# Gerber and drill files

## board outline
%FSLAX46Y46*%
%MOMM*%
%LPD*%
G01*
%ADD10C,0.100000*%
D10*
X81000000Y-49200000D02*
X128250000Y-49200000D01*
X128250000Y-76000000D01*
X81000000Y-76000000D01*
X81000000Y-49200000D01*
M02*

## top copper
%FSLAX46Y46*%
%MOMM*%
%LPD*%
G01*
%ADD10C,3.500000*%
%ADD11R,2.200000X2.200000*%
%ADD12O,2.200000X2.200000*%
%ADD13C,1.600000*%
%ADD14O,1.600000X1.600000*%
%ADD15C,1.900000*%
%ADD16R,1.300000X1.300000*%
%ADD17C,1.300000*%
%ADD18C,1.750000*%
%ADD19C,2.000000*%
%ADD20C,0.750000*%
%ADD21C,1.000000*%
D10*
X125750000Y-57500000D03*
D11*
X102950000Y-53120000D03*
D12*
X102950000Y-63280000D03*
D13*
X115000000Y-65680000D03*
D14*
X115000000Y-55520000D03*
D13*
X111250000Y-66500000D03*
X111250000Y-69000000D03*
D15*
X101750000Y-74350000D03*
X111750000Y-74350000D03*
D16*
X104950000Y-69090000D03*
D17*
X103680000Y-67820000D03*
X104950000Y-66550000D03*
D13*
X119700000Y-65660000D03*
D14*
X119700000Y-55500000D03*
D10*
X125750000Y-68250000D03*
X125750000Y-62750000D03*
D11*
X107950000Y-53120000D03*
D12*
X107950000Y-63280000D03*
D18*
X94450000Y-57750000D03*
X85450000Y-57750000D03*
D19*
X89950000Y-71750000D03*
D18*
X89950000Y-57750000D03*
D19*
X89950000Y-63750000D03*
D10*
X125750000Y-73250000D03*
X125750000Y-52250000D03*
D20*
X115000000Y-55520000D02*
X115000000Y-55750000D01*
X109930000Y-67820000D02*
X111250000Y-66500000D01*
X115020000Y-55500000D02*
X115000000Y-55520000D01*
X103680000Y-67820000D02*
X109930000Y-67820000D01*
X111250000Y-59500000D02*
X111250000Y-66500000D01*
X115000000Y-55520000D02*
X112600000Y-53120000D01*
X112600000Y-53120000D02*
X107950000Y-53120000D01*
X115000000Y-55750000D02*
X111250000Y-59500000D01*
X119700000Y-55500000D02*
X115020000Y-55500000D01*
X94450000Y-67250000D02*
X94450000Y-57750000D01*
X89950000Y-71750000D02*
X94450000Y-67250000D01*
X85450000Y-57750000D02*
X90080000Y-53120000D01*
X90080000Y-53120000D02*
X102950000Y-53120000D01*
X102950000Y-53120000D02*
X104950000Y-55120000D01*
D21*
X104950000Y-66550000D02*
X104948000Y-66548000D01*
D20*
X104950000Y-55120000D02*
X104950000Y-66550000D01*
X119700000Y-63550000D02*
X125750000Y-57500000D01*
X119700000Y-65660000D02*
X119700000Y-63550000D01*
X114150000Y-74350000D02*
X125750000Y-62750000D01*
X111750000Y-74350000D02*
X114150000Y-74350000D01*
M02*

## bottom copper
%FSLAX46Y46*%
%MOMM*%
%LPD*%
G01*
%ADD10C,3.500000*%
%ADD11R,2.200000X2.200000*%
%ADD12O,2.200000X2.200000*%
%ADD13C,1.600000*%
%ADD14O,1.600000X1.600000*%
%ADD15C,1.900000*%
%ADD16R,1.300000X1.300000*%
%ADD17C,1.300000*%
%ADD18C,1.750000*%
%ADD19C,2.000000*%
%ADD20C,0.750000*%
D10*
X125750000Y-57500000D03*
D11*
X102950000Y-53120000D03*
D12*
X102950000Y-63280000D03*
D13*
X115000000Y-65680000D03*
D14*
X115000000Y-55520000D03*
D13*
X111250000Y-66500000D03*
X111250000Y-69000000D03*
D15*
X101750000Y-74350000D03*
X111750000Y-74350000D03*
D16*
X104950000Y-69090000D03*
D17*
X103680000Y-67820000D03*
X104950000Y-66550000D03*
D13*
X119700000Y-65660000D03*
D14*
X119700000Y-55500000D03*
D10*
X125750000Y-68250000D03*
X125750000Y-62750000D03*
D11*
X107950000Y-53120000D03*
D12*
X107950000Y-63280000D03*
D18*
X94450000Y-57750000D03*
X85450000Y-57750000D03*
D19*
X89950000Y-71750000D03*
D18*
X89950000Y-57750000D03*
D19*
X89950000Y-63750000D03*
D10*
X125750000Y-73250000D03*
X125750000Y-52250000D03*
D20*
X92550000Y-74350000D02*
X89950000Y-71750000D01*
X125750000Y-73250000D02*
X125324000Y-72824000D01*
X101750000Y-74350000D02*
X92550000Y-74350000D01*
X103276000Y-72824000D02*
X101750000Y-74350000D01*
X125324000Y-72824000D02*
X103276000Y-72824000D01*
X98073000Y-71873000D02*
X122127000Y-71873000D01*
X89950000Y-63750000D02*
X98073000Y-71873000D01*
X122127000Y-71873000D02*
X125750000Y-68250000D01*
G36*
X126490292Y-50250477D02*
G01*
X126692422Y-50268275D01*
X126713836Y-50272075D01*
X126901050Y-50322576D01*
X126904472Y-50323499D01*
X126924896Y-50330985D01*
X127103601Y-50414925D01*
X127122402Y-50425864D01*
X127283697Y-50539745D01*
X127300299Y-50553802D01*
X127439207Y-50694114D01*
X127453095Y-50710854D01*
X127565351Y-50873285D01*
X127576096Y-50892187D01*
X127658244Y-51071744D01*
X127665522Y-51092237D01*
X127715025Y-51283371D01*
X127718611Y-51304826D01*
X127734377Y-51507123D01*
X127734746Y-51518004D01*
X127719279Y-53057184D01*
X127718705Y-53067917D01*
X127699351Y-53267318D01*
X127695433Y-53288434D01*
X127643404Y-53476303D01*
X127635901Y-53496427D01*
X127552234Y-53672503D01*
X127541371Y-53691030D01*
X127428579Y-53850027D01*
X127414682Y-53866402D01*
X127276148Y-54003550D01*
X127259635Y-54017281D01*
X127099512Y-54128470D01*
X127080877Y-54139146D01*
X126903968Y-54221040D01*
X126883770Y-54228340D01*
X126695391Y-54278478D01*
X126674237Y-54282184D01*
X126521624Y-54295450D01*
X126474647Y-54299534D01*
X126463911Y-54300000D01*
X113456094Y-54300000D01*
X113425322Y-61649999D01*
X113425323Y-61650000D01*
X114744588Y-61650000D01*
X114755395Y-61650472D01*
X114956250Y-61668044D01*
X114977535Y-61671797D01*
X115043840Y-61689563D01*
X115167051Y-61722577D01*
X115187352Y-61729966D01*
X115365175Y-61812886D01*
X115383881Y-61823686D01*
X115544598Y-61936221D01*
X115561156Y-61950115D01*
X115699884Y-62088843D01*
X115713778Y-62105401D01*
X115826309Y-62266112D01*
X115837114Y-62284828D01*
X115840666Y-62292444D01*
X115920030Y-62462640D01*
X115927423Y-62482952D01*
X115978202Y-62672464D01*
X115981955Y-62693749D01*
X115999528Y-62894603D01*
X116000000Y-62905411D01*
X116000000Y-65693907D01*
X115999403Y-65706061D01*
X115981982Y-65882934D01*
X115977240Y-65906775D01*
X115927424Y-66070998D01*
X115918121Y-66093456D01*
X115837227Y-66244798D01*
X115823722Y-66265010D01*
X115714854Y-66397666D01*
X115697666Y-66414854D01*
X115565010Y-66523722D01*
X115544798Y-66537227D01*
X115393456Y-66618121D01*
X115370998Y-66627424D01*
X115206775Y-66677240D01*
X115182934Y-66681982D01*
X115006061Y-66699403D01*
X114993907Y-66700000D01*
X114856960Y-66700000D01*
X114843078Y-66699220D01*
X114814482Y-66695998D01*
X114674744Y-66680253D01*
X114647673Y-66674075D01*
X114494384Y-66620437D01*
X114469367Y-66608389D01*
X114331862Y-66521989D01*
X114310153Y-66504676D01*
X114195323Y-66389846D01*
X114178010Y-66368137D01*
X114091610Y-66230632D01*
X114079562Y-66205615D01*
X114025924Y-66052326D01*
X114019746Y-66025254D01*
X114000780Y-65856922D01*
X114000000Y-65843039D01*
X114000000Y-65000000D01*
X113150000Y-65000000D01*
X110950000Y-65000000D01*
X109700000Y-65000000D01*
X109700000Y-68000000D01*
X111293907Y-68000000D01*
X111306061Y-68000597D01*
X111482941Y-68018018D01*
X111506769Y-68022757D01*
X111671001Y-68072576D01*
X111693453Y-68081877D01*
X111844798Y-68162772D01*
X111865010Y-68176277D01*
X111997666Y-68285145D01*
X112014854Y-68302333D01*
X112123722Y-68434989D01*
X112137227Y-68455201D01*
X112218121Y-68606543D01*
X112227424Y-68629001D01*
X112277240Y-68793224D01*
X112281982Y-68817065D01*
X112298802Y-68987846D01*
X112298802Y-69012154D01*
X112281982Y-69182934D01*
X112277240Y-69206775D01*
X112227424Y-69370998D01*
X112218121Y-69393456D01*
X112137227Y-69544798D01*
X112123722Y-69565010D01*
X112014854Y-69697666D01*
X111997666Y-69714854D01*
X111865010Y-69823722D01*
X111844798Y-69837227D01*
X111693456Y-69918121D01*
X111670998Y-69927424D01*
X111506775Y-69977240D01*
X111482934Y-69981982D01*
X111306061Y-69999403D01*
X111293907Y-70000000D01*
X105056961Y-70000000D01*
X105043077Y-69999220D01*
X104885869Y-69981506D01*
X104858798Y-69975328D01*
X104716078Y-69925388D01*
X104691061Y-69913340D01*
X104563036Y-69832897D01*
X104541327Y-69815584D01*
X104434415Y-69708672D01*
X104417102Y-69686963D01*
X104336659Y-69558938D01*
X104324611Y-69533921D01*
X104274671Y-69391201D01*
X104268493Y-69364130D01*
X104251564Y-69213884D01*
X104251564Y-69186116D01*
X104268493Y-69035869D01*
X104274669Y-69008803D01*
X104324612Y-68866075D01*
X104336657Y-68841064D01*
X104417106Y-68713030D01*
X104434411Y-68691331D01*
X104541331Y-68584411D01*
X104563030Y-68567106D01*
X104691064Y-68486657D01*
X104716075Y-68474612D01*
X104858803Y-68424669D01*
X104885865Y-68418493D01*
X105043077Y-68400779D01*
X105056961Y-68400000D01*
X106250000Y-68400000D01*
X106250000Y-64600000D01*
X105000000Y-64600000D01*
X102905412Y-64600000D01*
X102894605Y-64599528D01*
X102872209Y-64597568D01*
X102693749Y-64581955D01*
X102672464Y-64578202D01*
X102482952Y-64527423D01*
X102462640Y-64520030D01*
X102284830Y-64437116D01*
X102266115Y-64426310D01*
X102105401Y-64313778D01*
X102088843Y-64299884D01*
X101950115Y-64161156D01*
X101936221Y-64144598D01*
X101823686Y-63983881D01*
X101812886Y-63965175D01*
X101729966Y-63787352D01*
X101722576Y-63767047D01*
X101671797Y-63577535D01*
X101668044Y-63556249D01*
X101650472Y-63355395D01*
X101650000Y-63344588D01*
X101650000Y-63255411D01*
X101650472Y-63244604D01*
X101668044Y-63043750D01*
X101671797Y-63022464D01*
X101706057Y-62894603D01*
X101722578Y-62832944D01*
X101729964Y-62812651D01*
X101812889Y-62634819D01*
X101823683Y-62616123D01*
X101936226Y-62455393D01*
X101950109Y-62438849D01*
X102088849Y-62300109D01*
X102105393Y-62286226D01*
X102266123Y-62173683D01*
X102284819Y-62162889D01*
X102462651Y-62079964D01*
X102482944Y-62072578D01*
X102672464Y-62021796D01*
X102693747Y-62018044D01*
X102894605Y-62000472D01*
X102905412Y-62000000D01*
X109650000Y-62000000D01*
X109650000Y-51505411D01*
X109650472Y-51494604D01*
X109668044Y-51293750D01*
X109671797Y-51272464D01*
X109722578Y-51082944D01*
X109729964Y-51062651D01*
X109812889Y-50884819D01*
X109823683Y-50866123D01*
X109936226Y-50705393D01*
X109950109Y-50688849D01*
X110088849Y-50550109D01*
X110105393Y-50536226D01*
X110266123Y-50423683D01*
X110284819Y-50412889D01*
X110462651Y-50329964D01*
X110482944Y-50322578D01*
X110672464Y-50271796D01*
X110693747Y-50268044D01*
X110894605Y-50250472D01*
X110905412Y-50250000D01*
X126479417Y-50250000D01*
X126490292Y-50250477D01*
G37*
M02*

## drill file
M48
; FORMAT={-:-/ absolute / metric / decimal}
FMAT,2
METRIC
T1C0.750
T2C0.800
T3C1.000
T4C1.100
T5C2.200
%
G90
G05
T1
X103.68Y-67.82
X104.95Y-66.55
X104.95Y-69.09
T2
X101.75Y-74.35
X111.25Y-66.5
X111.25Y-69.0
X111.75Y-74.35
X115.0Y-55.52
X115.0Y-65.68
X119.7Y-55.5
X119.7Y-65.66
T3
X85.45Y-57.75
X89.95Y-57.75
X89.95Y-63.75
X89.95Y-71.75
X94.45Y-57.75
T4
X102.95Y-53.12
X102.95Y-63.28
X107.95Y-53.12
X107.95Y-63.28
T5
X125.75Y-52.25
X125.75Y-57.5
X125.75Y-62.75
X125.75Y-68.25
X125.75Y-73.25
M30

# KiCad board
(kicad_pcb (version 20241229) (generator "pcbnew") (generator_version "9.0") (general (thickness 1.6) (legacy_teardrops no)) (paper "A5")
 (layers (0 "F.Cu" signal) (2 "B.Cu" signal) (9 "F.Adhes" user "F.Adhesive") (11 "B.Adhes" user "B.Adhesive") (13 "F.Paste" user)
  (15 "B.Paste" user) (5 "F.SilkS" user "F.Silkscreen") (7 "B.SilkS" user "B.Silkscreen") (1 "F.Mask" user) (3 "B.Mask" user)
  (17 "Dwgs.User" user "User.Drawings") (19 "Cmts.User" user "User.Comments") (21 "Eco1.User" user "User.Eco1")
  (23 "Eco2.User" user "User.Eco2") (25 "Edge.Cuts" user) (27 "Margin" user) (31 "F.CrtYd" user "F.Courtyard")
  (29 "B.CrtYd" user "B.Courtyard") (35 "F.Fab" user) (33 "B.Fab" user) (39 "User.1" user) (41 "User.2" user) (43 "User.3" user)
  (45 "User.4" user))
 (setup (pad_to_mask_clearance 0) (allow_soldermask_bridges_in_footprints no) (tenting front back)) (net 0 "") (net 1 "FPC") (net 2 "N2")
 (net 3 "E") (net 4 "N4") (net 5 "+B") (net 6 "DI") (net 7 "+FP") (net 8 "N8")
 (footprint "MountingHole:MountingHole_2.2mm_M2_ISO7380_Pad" (layer "F.Cu") (at 125.75 57.5 90)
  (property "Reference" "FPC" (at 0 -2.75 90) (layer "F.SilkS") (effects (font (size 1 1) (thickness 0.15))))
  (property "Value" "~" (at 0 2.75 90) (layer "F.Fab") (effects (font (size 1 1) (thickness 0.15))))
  (pad "1" thru_hole circle (at 0 0 90) (size 3.5 3.5) (drill 2.2) (layers "*.Cu" "*.Mask") (remove_unused_layers no) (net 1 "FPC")))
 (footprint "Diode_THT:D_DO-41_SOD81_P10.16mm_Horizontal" (layer "F.Cu") (at 102.95 53.12 -90)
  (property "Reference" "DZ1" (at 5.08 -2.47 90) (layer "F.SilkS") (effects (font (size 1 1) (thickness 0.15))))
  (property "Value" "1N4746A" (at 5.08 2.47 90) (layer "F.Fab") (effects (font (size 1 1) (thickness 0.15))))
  (pad "1" thru_hole rect (at 0 0 270) (size 2.2 2.2) (drill 1.1) (layers "*.Cu" "*.Mask") (remove_unused_layers no) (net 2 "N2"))
  (pad "2" thru_hole oval (at 10.16 0 270) (size 2.2 2.2) (drill 1.1) (layers "*.Cu" "*.Mask") (remove_unused_layers no) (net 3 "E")))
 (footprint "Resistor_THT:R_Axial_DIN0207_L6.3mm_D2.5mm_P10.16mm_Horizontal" (layer "F.Cu") (at 115 65.68 90)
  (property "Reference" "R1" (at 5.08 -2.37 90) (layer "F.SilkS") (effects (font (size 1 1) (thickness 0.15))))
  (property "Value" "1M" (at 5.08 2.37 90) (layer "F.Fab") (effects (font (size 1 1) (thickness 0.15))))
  (pad "1" thru_hole circle (at 0 0 90) (size 1.6 1.6) (drill 0.8) (layers "*.Cu" "*.Mask") (remove_unused_layers no) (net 3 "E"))
  (pad "2" thru_hole oval (at 10.16 0 90) (size 1.6 1.6) (drill 0.8) (layers "*.Cu" "*.Mask") (remove_unused_layers no) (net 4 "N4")))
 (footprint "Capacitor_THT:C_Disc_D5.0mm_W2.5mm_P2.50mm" (layer "F.Cu") (at 111.25 66.5 -90)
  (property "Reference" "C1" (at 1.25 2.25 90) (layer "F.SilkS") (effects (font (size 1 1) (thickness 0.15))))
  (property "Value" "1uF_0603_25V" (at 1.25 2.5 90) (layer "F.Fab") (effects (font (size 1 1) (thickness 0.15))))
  (pad "1" thru_hole circle (at 0 0 270) (size 1.6 1.6) (drill 0.8) (layers "*.Cu" "*.Mask") (remove_unused_layers no) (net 4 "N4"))
  (pad "2" thru_hole circle (at 2.5 0 270) (size 1.6 1.6) (drill 0.8) (layers "*.Cu" "*.Mask") (remove_unused_layers no) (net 3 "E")))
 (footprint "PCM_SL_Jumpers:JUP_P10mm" (layer "F.Cu") (at 106.75 74.35)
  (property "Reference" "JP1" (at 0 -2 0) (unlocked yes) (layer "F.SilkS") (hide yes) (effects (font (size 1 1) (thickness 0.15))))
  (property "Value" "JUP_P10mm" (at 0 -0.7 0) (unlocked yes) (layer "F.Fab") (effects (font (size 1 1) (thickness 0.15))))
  (pad "1" thru_hole circle (at -5 0) (size 1.9 1.9) (drill 0.8) (layers "*.Cu" "*.Mask") (remove_unused_layers no) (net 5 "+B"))
  (pad "2" thru_hole circle (at 5 0) (size 1.9 1.9) (drill 0.8) (layers "*.Cu" "*.Mask") (remove_unused_layers no) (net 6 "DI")))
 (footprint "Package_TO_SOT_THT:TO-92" (layer "F.Cu") (at 104.95 69.09 90)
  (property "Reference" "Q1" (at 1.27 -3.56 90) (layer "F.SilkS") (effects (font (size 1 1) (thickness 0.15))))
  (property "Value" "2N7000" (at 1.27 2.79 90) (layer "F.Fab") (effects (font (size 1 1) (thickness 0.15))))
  (pad "1" thru_hole rect (at 0 0 90) (size 1.3 1.3) (drill 0.75) (layers "*.Cu" "*.Mask") (remove_unused_layers no) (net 3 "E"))
  (pad "2" thru_hole circle (at 1.27 -1.27 90) (size 1.3 1.3) (drill 0.75) (layers "*.Cu" "*.Mask") (remove_unused_layers no) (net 4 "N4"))
  (pad "3" thru_hole circle (at 2.54 0 90) (size 1.3 1.3) (drill 0.75) (layers "*.Cu" "*.Mask") (remove_unused_layers no) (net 2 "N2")))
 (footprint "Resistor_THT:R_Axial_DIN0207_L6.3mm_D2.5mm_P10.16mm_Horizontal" (layer "F.Cu") (at 119.7 65.66 90)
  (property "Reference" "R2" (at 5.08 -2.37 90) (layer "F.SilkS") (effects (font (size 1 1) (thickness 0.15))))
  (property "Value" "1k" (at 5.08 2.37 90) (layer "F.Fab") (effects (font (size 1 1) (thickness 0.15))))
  (pad "1" thru_hole circle (at 0 0 90) (size 1.6 1.6) (drill 0.8) (layers "*.Cu" "*.Mask") (remove_unused_layers no) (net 1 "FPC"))
  (pad "2" thru_hole oval (at 10.16 0 90) (size 1.6 1.6) (drill 0.8) (layers "*.Cu" "*.Mask") (remove_unused_layers no) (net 4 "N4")))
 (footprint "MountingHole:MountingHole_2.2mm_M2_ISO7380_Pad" (layer "F.Cu") (at 125.75 68.25 90)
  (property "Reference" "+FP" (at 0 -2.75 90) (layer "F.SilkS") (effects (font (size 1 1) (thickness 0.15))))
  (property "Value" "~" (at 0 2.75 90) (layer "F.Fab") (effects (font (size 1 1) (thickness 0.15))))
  (pad "1" thru_hole circle (at 0 0 90) (size 3.5 3.5) (drill 2.2) (layers "*.Cu" "*.Mask") (remove_unused_layers no) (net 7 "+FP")))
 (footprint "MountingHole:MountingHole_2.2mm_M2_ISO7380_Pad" (layer "F.Cu") (at 125.75 62.75 90)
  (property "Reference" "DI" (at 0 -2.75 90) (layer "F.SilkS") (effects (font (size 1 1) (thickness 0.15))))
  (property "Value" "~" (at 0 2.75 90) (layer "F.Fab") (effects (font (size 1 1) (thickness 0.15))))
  (pad "1" thru_hole circle (at 0 0 90) (size 3.5 3.5) (drill 2.2) (layers "*.Cu" "*.Mask") (remove_unused_layers no) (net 6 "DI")))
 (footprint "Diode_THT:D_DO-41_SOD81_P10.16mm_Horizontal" (layer "F.Cu") (at 107.95 53.12 -90)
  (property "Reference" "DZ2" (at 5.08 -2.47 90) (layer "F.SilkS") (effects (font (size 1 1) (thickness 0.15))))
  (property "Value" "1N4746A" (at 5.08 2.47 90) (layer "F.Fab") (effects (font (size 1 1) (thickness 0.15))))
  (pad "1" thru_hole rect (at 0 0 270) (size 2.2 2.2) (drill 1.1) (layers "*.Cu" "*.Mask") (remove_unused_layers no) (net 4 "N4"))
  (pad "2" thru_hole oval (at 10.16 0 270) (size 2.2 2.2) (drill 1.1) (layers "*.Cu" "*.Mask") (remove_unused_layers no) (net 3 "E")))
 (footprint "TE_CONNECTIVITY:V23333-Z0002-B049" (layer "F.Cu") (at 89.95 63.75)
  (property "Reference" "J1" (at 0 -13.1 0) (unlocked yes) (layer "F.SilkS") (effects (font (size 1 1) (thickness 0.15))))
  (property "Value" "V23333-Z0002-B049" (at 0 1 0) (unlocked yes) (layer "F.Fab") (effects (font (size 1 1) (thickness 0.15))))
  (pad "1" thru_hole circle (at 4.5 -6) (size 1.75 1.75) (drill 1) (layers "*.Cu" "*.Mask") (remove_unused_layers no) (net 5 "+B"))
  (pad "2" thru_hole circle (at -4.5 -6) (size 1.75 1.75) (drill 1) (layers "*.Cu" "*.Mask") (remove_unused_layers no) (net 2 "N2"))
  (pad "3" thru_hole circle (at 0 8) (size 2 2) (drill 1) (layers "*.Cu" "*.Mask") (remove_unused_layers no) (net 5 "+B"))
  (pad "4" thru_hole circle (at 0 -6) (size 1.75 1.75) (drill 1) (layers "*.Cu" "*.Mask") (remove_unused_layers no) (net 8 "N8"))
  (pad "5" thru_hole circle (at 0 0) (size 2 2) (drill 1) (layers "*.Cu" "*.Mask") (remove_unused_layers no) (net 7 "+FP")))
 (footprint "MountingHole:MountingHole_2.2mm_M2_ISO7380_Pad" (layer "F.Cu") (at 125.75 73.25 90)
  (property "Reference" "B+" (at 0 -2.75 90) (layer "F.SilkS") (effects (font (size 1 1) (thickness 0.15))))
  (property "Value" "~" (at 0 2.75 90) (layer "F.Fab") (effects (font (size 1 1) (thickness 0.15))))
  (pad "1" thru_hole circle (at 0 0 90) (size 3.5 3.5) (drill 2.2) (layers "*.Cu" "*.Mask") (remove_unused_layers no) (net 5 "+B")))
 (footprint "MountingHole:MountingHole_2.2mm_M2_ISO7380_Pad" (layer "F.Cu") (at 125.75 52.25 90)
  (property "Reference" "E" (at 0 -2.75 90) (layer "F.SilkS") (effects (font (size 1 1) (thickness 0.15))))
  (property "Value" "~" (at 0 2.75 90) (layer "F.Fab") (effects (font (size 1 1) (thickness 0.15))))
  (pad "1" thru_hole circle (at 0 0 90) (size 3.5 3.5) (drill 2.2) (layers "*.Cu" "*.Mask") (remove_unused_layers no) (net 3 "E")))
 (gr_rect (start 81 49.2) (end 128.25 76) (stroke (width 0.1) (type default)) (fill no) (layer "Edge.Cuts"))
 (segment (start 115 55.52) (end 115 55.75) (width 0.75) (layer "F.Cu") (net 4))
 (segment (start 109.93 67.82) (end 111.25 66.5) (width 0.75) (layer "F.Cu") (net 4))
 (segment (start 115.02 55.5) (end 115 55.52) (width 0.75) (layer "F.Cu") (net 4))
 (segment (start 103.68 67.82) (end 109.93 67.82) (width 0.75) (layer "F.Cu") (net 4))
 (segment (start 111.25 59.5) (end 111.25 66.5) (width 0.75) (layer "F.Cu") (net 4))
 (segment (start 115 55.52) (end 112.6 53.12) (width 0.75) (layer "F.Cu") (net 4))
 (segment (start 112.6 53.12) (end 107.95 53.12) (width 0.75) (layer "F.Cu") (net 4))
 (segment (start 115 55.75) (end 111.25 59.5) (width 0.75) (layer "F.Cu") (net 4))
 (segment (start 119.7 55.5) (end 115.02 55.5) (width 0.75) (layer "F.Cu") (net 4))
 (segment (start 94.45 67.25) (end 94.45 57.75) (width 0.75) (layer "F.Cu") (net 5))
 (segment (start 89.95 71.75) (end 94.45 67.25) (width 0.75) (layer "F.Cu") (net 5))
 (segment (start 92.55 74.35) (end 89.95 71.75) (width 0.75) (layer "B.Cu") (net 5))
 (segment (start 125.75 73.25) (end 125.324 72.824) (width 0.75) (layer "B.Cu") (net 5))
 (segment (start 101.75 74.35) (end 92.55 74.35) (width 0.75) (layer "B.Cu") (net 5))
 (segment (start 103.276 72.824) (end 101.75 74.35) (width 0.75) (layer "B.Cu") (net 5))
 (segment (start 125.324 72.824) (end 103.276 72.824) (width 0.75) (layer "B.Cu") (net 5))
 (segment (start 85.45 57.75) (end 90.08 53.12) (width 0.75) (layer "F.Cu") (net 2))
 (segment (start 90.08 53.12) (end 102.95 53.12) (width 0.75) (layer "F.Cu") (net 2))
 (segment (start 102.95 53.12) (end 104.95 55.12) (width 0.75) (layer "F.Cu") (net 2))
 (segment (start 104.95 66.55) (end 104.948 66.548) (width 1) (layer "F.Cu") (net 2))
 (segment (start 104.95 55.12) (end 104.95 66.55) (width 0.75) (layer "F.Cu") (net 2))
 (segment (start 98.073 71.873) (end 122.127 71.873) (width 0.75) (layer "B.Cu") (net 7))
 (segment (start 89.95 63.75) (end 98.073 71.873) (width 0.75) (layer "B.Cu") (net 7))
 (segment (start 122.127 71.873) (end 125.75 68.25) (width 0.75) (layer "B.Cu") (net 7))
 (segment (start 119.7 63.55) (end 125.75 57.5) (width 0.75) (layer "F.Cu") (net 1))
 (segment (start 119.7 65.66) (end 119.7 63.55) (width 0.75) (layer "F.Cu") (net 1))
 (segment (start 114.15 74.35) (end 125.75 62.75) (width 0.75) (layer "F.Cu") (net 6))
 (segment (start 111.75 74.35) (end 114.15 74.35) (width 0.75) (layer "F.Cu") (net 6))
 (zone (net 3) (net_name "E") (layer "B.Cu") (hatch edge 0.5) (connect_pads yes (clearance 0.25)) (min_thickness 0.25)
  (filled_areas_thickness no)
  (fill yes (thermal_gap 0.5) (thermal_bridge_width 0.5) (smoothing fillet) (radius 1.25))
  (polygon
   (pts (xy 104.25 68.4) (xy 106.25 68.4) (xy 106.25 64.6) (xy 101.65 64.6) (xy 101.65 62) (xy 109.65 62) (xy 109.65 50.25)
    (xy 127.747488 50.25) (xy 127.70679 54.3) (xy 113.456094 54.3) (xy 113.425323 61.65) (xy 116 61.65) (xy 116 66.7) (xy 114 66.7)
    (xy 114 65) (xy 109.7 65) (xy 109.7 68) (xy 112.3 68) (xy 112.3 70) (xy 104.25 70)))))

